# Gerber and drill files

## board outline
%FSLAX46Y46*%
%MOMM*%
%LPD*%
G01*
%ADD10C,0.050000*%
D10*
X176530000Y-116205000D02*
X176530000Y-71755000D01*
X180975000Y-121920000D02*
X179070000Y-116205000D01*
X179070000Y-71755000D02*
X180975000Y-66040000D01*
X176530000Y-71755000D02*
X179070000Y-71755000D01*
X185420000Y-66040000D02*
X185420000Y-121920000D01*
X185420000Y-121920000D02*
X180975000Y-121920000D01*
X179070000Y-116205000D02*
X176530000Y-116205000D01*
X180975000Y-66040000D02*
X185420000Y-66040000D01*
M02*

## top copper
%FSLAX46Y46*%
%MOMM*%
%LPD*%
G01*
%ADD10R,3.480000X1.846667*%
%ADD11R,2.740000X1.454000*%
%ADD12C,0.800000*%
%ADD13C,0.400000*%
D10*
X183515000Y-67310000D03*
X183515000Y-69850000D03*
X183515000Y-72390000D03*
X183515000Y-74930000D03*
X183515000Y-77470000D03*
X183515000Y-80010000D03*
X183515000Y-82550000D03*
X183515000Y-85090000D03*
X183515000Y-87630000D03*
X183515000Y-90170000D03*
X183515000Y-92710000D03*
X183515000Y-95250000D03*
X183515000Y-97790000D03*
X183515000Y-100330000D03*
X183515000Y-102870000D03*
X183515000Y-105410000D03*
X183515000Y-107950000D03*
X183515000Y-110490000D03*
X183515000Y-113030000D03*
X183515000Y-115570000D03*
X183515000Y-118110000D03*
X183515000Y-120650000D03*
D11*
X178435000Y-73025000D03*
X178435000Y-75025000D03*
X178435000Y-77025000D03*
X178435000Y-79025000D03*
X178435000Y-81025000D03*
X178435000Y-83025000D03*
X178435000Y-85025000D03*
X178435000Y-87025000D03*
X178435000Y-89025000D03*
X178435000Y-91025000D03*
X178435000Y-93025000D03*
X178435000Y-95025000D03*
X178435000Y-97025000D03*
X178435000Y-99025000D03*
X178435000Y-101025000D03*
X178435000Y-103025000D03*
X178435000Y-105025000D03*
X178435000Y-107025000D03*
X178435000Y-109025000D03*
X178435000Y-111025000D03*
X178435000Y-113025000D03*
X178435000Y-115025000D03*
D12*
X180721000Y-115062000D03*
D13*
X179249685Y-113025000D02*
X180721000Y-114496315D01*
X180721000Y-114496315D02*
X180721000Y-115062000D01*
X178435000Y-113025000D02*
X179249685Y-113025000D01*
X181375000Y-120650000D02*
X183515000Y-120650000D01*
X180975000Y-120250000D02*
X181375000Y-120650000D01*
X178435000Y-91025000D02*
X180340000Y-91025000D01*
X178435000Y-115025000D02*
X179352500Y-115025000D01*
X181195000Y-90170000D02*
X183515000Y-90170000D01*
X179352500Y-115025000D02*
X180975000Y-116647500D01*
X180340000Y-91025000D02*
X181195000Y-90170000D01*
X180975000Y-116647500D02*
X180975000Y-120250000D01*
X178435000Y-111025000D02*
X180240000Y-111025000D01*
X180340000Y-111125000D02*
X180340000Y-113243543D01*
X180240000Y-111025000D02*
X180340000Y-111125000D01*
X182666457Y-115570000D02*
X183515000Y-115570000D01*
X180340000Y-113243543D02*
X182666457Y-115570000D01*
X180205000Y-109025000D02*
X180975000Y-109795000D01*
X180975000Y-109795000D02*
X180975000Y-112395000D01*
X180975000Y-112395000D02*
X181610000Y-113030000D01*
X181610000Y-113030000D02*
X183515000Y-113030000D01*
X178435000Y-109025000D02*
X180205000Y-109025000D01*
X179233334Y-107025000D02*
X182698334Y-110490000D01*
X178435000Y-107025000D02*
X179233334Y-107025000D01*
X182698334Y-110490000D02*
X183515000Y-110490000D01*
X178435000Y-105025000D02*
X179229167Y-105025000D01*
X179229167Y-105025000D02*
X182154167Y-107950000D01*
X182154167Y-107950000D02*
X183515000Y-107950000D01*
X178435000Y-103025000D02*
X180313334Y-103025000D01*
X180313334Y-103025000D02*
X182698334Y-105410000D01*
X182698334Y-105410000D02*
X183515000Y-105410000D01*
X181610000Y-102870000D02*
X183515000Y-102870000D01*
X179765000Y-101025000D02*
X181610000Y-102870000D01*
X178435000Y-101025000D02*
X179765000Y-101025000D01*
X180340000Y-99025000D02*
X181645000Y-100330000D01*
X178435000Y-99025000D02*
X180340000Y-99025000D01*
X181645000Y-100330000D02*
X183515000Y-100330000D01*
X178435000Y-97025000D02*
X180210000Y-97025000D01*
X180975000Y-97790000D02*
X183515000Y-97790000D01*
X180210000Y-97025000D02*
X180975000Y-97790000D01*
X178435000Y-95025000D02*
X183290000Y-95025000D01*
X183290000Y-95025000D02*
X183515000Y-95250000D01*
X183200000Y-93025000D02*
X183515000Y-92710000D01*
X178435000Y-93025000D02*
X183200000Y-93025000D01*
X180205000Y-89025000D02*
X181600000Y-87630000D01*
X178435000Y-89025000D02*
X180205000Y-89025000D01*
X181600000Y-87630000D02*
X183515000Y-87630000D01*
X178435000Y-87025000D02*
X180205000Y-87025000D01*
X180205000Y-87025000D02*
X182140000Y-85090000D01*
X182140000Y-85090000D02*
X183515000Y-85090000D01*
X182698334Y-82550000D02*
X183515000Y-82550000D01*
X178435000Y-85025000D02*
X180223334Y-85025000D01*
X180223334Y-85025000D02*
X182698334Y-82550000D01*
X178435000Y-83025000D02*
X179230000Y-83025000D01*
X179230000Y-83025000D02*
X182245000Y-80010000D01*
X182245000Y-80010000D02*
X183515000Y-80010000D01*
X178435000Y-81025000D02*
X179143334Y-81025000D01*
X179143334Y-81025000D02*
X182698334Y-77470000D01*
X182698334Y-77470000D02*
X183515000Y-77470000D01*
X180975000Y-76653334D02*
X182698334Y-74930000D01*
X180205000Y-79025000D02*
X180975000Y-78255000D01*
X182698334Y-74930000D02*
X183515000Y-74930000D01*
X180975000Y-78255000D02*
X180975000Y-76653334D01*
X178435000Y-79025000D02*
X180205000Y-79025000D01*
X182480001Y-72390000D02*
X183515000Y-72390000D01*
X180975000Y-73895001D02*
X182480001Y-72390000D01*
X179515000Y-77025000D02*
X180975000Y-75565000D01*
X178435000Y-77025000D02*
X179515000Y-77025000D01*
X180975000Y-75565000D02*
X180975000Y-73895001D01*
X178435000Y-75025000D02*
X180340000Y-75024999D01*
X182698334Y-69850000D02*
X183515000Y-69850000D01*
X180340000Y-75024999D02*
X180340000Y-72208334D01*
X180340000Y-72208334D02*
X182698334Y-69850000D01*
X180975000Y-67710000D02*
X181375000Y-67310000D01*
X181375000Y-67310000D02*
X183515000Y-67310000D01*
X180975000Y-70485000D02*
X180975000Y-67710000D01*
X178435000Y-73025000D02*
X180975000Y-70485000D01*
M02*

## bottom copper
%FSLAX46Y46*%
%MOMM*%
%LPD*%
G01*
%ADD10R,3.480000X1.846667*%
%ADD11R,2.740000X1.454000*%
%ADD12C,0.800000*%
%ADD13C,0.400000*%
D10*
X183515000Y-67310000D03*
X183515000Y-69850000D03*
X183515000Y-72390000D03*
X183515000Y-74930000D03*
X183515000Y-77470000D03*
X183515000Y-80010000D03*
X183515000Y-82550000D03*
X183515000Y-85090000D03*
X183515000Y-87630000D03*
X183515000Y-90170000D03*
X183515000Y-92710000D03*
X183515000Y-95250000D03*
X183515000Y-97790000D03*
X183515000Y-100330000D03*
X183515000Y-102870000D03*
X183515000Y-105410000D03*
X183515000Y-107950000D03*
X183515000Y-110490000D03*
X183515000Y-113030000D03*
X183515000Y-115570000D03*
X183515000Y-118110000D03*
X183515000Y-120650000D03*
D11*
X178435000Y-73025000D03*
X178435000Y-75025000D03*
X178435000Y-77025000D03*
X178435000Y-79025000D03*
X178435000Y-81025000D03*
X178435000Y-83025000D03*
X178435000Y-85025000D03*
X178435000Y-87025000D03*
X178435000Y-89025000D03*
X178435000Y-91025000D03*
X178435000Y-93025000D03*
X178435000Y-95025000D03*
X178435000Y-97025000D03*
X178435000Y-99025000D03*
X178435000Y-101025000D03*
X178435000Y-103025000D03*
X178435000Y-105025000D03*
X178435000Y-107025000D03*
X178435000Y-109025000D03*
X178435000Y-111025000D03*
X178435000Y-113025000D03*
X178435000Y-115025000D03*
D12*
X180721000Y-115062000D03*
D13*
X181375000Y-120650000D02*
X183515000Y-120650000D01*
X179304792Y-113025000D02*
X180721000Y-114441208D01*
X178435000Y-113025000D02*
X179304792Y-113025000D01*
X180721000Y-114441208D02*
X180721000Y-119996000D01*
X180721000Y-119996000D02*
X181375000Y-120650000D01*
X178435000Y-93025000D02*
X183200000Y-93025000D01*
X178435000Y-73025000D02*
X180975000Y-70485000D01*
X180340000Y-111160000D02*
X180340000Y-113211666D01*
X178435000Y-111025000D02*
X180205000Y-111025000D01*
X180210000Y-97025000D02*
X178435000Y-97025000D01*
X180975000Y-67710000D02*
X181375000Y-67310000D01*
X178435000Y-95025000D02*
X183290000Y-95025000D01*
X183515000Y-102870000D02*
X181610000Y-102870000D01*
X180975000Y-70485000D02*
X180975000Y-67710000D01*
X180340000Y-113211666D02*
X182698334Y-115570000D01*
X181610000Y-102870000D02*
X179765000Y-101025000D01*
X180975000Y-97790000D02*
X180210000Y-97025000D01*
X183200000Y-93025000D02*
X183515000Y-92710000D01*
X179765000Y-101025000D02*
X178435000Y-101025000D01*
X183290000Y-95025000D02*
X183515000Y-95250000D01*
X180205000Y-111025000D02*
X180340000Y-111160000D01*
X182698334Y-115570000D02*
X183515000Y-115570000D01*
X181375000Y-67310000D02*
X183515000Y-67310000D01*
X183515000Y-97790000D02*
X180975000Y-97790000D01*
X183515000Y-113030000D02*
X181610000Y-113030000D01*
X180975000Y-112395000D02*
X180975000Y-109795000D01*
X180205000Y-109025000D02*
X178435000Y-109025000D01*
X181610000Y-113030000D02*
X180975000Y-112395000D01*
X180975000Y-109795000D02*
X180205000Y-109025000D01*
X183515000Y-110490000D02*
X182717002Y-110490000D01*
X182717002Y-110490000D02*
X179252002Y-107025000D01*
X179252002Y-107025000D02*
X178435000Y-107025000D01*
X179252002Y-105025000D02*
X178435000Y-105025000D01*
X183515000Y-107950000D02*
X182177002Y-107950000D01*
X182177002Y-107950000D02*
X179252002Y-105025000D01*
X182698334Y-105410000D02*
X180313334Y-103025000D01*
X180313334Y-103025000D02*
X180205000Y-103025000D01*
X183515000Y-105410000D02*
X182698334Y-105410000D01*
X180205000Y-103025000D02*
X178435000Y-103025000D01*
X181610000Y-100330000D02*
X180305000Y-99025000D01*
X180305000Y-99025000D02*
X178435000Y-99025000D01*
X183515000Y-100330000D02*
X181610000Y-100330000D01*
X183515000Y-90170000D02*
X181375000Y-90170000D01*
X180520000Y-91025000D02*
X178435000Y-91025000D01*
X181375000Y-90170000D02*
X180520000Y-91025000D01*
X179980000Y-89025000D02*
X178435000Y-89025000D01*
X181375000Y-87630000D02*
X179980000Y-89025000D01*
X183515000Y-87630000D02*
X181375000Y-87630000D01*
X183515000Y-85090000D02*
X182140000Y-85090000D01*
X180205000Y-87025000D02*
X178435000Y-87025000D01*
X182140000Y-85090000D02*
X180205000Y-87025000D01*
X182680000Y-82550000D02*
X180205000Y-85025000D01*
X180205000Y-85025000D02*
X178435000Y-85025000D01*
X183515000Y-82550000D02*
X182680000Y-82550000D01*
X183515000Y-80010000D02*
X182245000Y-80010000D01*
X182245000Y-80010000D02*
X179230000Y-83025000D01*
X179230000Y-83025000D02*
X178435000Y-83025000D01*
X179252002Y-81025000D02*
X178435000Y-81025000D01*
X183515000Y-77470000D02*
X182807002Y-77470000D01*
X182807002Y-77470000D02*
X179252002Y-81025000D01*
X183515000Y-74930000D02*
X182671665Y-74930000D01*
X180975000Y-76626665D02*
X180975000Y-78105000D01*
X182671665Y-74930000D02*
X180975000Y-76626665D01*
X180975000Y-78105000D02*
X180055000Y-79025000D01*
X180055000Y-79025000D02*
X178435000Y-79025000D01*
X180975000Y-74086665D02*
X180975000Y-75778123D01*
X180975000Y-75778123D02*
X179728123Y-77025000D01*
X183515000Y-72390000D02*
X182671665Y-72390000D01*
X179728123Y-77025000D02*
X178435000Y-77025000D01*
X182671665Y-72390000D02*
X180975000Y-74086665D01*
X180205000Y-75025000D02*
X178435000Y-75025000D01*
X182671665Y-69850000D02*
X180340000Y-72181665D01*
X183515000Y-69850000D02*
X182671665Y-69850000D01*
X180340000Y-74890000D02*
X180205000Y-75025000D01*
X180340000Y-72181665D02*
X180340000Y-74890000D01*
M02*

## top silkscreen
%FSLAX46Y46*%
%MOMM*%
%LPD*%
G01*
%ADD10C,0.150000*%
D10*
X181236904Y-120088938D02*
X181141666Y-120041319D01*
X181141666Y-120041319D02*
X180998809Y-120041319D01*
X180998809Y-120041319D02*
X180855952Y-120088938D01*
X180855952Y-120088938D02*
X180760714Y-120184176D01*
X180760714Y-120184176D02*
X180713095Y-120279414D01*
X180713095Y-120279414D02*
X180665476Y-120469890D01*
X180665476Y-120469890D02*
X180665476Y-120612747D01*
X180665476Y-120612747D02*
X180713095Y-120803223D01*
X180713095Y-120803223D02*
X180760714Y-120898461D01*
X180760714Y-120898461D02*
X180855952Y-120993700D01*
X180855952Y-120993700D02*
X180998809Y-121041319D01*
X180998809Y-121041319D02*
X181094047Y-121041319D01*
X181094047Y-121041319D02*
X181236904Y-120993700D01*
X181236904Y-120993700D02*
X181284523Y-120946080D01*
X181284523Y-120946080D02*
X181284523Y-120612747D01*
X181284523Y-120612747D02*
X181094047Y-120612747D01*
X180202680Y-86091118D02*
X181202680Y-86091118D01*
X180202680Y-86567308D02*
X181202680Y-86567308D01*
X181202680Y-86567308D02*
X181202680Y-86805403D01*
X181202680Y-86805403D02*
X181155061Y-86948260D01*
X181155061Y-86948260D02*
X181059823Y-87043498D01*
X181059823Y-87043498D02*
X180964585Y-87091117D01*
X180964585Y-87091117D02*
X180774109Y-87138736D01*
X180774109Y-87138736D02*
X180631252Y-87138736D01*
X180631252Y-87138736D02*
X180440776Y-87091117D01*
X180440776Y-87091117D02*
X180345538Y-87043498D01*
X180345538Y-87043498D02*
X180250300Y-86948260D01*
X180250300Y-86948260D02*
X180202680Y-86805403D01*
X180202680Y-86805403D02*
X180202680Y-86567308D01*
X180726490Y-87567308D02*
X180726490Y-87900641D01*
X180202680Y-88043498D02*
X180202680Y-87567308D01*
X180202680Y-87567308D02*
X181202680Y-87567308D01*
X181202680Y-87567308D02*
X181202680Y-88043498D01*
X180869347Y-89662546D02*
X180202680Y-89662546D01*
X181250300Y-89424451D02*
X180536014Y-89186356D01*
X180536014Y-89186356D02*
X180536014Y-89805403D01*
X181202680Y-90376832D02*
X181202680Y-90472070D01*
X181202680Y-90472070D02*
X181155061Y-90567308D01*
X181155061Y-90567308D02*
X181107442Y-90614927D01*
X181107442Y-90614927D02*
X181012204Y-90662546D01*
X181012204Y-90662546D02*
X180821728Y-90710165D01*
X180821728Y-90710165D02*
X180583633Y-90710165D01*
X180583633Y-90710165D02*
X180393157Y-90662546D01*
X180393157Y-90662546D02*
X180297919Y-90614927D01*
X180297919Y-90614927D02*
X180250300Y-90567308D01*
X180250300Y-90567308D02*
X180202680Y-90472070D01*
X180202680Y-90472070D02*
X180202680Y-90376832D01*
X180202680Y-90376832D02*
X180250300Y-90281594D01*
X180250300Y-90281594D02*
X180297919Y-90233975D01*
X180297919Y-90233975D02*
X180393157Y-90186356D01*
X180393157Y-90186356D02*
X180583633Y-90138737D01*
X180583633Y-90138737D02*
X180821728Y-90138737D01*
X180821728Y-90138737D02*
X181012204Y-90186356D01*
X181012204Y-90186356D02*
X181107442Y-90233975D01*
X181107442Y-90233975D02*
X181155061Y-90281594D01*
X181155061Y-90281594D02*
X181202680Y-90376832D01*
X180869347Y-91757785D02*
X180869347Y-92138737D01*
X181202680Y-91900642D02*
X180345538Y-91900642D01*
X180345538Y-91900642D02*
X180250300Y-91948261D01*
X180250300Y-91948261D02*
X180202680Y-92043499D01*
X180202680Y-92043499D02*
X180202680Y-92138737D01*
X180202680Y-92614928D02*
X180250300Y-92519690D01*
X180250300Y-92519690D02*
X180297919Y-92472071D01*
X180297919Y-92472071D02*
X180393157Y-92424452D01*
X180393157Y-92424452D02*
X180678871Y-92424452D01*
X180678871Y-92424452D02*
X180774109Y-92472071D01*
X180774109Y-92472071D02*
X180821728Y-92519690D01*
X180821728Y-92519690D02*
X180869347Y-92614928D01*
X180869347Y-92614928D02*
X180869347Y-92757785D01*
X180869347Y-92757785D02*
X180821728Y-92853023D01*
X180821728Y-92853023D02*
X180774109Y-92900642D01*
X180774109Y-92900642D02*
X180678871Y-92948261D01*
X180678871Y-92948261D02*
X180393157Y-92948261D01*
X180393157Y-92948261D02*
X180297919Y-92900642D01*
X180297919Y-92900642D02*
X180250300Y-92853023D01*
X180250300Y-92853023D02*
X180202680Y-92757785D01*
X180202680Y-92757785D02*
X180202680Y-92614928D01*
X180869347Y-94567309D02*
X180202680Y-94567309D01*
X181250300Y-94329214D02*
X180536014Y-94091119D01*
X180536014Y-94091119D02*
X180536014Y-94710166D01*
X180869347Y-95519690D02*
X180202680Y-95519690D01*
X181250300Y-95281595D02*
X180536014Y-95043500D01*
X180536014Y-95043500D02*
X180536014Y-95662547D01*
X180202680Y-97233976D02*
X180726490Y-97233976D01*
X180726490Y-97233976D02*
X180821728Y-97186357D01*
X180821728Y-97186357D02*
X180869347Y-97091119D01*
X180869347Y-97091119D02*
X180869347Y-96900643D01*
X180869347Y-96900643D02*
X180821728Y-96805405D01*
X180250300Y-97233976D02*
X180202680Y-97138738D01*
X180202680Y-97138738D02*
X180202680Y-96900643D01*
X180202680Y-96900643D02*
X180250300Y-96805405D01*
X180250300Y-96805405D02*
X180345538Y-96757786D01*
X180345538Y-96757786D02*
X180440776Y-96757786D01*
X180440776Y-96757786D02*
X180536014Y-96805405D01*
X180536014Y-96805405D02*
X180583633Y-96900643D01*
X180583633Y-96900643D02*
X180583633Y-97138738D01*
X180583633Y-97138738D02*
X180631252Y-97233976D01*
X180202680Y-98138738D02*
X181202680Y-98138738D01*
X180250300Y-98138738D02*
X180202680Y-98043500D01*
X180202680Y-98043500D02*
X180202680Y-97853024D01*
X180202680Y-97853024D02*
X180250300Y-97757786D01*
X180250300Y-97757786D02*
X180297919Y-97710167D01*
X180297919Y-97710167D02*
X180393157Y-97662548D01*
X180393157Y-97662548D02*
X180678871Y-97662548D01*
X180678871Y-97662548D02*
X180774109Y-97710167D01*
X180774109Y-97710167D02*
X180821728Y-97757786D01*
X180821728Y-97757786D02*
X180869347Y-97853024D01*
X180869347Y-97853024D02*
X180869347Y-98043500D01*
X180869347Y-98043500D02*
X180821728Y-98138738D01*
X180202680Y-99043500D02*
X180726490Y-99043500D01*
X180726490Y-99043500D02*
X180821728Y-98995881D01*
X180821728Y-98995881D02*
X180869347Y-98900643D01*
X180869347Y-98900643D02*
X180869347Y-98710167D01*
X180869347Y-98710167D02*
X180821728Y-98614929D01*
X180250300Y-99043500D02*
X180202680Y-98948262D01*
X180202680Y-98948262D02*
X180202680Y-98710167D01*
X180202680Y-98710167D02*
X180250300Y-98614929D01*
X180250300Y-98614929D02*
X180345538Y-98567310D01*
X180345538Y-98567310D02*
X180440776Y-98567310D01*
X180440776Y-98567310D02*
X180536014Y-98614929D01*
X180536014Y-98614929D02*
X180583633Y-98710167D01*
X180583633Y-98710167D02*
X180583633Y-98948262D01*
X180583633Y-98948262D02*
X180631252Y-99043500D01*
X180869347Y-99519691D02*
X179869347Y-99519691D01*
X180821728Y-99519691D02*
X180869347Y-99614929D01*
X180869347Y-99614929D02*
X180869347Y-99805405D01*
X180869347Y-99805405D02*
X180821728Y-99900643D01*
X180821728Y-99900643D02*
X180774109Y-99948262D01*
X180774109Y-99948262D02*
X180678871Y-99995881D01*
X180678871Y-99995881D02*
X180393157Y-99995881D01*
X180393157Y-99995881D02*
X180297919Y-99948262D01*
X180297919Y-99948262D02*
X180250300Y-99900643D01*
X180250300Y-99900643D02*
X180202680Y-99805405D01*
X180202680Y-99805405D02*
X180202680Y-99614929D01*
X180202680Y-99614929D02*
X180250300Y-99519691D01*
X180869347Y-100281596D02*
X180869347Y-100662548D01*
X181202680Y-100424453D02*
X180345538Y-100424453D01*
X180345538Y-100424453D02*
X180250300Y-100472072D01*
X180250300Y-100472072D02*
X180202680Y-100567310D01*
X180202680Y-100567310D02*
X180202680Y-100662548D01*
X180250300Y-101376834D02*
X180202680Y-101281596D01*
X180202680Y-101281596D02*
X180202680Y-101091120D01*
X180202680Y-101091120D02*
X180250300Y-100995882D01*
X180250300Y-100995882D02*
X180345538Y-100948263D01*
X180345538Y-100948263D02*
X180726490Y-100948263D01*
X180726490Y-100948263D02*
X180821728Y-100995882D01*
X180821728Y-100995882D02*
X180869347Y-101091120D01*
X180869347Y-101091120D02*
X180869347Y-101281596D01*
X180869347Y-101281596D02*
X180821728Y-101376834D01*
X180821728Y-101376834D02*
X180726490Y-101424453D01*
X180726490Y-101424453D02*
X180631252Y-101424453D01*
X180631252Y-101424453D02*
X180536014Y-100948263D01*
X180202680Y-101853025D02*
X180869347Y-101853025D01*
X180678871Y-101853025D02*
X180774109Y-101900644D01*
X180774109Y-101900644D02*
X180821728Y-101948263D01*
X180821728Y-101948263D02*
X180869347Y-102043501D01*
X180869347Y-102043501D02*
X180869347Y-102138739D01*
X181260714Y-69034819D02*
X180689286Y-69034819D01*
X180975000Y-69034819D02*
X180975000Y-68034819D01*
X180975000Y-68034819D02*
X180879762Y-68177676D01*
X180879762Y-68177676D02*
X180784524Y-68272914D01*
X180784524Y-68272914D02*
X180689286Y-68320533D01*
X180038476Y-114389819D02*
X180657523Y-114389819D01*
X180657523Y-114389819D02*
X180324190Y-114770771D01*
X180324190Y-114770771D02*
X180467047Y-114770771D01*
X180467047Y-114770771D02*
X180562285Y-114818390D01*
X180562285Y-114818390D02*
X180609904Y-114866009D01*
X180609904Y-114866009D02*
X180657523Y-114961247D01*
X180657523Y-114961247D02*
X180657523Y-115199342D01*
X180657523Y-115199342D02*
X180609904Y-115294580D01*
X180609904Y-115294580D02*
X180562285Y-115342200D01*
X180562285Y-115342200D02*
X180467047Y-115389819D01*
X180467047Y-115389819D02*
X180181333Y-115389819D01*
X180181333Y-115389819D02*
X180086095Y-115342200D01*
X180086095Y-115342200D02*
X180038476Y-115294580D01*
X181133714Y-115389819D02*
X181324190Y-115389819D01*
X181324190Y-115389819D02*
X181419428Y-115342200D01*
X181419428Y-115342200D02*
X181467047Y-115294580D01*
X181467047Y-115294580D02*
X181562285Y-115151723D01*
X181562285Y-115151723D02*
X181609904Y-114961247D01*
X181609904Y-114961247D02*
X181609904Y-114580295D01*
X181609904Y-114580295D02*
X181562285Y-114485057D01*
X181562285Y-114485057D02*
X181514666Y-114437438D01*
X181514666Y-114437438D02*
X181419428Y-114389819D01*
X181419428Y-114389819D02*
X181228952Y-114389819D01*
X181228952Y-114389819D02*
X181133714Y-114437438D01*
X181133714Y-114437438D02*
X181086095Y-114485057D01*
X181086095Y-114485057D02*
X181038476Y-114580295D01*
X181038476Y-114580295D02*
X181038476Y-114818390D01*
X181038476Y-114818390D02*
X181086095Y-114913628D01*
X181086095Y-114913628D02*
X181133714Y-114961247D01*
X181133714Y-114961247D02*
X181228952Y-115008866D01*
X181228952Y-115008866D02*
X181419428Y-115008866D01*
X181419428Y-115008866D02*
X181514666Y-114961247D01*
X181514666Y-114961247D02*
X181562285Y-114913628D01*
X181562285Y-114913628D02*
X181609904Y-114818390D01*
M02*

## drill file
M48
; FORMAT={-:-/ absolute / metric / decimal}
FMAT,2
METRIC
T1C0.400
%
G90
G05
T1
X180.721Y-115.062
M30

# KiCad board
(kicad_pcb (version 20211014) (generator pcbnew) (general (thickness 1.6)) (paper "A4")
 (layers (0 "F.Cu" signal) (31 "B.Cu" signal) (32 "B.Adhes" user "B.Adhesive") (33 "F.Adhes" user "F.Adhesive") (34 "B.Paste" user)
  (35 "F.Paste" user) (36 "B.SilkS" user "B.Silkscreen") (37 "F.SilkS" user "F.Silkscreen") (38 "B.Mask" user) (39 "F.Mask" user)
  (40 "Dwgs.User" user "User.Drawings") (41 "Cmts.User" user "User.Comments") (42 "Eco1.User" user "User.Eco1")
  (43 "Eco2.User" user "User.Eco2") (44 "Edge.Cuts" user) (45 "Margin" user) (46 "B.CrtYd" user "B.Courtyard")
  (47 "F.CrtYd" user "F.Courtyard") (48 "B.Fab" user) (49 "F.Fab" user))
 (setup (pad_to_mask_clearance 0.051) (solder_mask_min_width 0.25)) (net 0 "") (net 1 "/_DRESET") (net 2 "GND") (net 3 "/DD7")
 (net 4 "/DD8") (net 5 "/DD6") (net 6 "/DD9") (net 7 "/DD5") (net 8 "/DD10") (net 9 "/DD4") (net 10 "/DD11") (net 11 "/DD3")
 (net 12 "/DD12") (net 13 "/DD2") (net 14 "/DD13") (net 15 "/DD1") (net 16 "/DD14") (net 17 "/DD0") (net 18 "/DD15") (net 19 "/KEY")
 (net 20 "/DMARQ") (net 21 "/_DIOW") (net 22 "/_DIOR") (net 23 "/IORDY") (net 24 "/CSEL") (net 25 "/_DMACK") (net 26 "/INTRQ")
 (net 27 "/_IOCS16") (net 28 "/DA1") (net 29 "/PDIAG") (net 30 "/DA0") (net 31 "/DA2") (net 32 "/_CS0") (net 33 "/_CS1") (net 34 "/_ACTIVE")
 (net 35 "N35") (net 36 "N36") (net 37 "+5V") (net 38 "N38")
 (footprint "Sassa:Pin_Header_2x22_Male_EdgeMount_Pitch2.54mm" (layer "B.Cu") (at 183.515 67.31 -90)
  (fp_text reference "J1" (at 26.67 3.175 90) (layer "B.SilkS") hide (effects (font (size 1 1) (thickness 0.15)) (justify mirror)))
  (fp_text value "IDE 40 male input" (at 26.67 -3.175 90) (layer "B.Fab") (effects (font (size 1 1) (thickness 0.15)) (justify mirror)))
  (pad "1" smd rect locked (at 0 0 270) (size 1.846667 3.48) (layers "F.Cu" "F.Paste" "F.Mask") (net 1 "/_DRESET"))
  (pad "2" smd rect locked (at 0 0 270) (size 1.846667 3.48) (layers "B.Cu" "B.Paste" "B.Mask") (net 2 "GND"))
  (pad "3" smd rect locked (at 2.54 0 270) (size 1.846667 3.48) (layers "F.Cu" "F.Paste" "F.Mask") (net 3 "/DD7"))
  (pad "4" smd rect locked (at 2.54 0 270) (size 1.846667 3.48) (layers "B.Cu" "B.Paste" "B.Mask") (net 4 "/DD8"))
  (pad "5" smd rect locked (at 5.08 0 270) (size 1.846667 3.48) (layers "F.Cu" "F.Paste" "F.Mask") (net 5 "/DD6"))
  (pad "6" smd rect locked (at 5.08 0 270) (size 1.846667 3.48) (layers "B.Cu" "B.Paste" "B.Mask") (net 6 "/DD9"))
  (pad "7" smd rect locked (at 7.62 0 270) (size 1.846667 3.48) (layers "F.Cu" "F.Paste" "F.Mask") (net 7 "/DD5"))
  (pad "8" smd rect locked (at 7.62 0 270) (size 1.846667 3.48) (layers "B.Cu" "B.Paste" "B.Mask") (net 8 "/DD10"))
  (pad "9" smd rect locked (at 10.16 0 270) (size 1.846667 3.48) (layers "F.Cu" "F.Paste" "F.Mask") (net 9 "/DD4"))
  (pad "10" smd rect locked (at 10.16 0 270) (size 1.846667 3.48) (layers "B.Cu" "B.Paste" "B.Mask") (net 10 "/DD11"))
  (pad "11" smd rect locked (at 12.7 0 270) (size 1.846667 3.48) (layers "F.Cu" "F.Paste" "F.Mask") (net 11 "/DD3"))
  (pad "12" smd rect locked (at 12.7 0 270) (size 1.846667 3.48) (layers "B.Cu" "B.Paste" "B.Mask") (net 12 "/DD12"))
  (pad "13" smd rect locked (at 15.24 0 270) (size 1.846667 3.48) (layers "F.Cu" "F.Paste" "F.Mask") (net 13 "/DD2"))
  (pad "14" smd rect locked (at 15.24 0 270) (size 1.846667 3.48) (layers "B.Cu" "B.Paste" "B.Mask") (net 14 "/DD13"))
  (pad "15" smd rect locked (at 17.78 0 270) (size 1.846667 3.48) (layers "F.Cu" "F.Paste" "F.Mask") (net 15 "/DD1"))
  (pad "16" smd rect locked (at 17.78 0 270) (size 1.846667 3.48) (layers "B.Cu" "B.Paste" "B.Mask") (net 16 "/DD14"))
  (pad "17" smd rect locked (at 20.32 0 270) (size 1.846667 3.48) (layers "F.Cu" "F.Paste" "F.Mask") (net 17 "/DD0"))
  (pad "18" smd rect locked (at 20.32 0 270) (size 1.846667 3.48) (layers "B.Cu" "B.Paste" "B.Mask") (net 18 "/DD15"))
  (pad "19" smd rect locked (at 22.86 0 270) (size 1.846667 3.48) (layers "F.Cu" "F.Paste" "F.Mask") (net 2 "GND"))
  (pad "20" smd rect locked (at 22.86 0 270) (size 1.846667 3.48) (layers "B.Cu" "B.Paste" "B.Mask") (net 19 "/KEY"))
  (pad "21" smd rect locked (at 25.4 0 270) (size 1.846667 3.48) (layers "F.Cu" "F.Paste" "F.Mask") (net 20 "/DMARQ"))
  (pad "22" smd rect locked (at 25.4 0 270) (size 1.846667 3.48) (layers "B.Cu" "B.Paste" "B.Mask") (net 2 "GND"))
  (pad "23" smd rect locked (at 27.94 0 270) (size 1.846667 3.48) (layers "F.Cu" "F.Paste" "F.Mask") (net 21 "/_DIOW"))
  (pad "24" smd rect locked (at 27.94 0 270) (size 1.846667 3.48) (layers "B.Cu" "B.Paste" "B.Mask") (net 2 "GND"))
  (pad "25" smd rect locked (at 30.48 0 270) (size 1.846667 3.48) (layers "F.Cu" "F.Paste" "F.Mask") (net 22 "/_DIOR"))
  (pad "26" smd rect locked (at 30.48 0 270) (size 1.846667 3.48) (layers "B.Cu" "B.Paste" "B.Mask") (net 2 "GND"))
  (pad "27" smd rect locked (at 33.02 0 270) (size 1.846667 3.48) (layers "F.Cu" "F.Paste" "F.Mask") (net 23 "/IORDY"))
  (pad "28" smd rect locked (at 33.02 0 270) (size 1.846667 3.48) (layers "B.Cu" "B.Paste" "B.Mask") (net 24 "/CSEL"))
  (pad "29" smd rect locked (at 35.56 0 270) (size 1.846667 3.48) (layers "F.Cu" "F.Paste" "F.Mask") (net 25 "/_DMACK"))
  (pad "30" smd rect locked (at 35.56 0 270) (size 1.846667 3.48) (layers "B.Cu" "B.Paste" "B.Mask") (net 2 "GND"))
  (pad "31" smd rect locked (at 38.1 0 270) (size 1.846667 3.48) (layers "F.Cu" "F.Paste" "F.Mask") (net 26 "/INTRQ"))
  (pad "32" smd rect locked (at 38.1 0 270) (size 1.846667 3.48) (layers "B.Cu" "B.Paste" "B.Mask") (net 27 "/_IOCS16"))
  (pad "33" smd rect locked (at 40.64 0 270) (size 1.846667 3.48) (layers "F.Cu" "F.Paste" "F.Mask") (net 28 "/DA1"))
  (pad "34" smd rect locked (at 40.64 0 270) (size 1.846667 3.48) (layers "B.Cu" "B.Paste" "B.Mask") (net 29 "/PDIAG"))
  (pad "35" smd rect locked (at 43.18 0 270) (size 1.846667 3.48) (layers "F.Cu" "F.Paste" "F.Mask") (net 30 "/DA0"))
  (pad "36" smd rect locked (at 43.18 0 270) (size 1.846667 3.48) (layers "B.Cu" "B.Paste" "B.Mask") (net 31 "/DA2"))
  (pad "37" smd rect locked (at 45.72 0 270) (size 1.846667 3.48) (layers "F.Cu" "F.Paste" "F.Mask") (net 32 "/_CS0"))
  (pad "38" smd rect locked (at 45.72 0 270) (size 1.846667 3.48) (layers "B.Cu" "B.Paste" "B.Mask") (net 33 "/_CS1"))
  (pad "39" smd rect locked (at 48.26 0 270) (size 1.846667 3.48) (layers "F.Cu" "F.Paste" "F.Mask") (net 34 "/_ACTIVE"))
  (pad "40" smd rect locked (at 48.26 0 270) (size 1.846667 3.48) (layers "B.Cu" "B.Paste" "B.Mask") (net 2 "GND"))
  (pad "41" smd rect locked (at 50.8 0 270) (size 1.846667 3.48) (layers "F.Cu" "F.Paste" "F.Mask") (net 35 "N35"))
  (pad "42" smd rect locked (at 50.8 0 270) (size 1.846667 3.48) (layers "B.Cu" "B.Paste" "B.Mask") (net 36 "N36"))
  (pad "43" smd rect locked (at 53.34 0 270) (size 1.846667 3.48) (layers "F.Cu" "F.Paste" "F.Mask") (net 2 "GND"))
  (pad "44" smd rect locked (at 53.34 0 270) (size 1.846667 3.48) (layers "B.Cu" "B.Paste" "B.Mask") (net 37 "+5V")))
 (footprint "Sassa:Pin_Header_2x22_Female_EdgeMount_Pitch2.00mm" (layer "B.Cu") (at 178.435 73.025 90)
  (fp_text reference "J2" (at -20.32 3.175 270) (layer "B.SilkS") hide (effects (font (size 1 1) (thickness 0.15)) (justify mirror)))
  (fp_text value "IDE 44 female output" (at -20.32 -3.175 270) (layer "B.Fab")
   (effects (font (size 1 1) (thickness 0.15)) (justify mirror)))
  (pad "1" smd rect locked (at 0 0 90) (size 1.454 2.74) (layers "F.Cu" "F.Paste" "F.Mask") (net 1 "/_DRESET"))
  (pad "2" smd rect locked (at 0 0 90) (size 1.454 2.74) (layers "B.Cu" "B.Paste" "B.Mask") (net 2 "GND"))
  (pad "3" smd rect locked (at -2 0 90) (size 1.454 2.74) (layers "F.Cu" "F.Paste" "F.Mask") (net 3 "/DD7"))
  (pad "4" smd rect locked (at -2 0 90) (size 1.454 2.74) (layers "B.Cu" "B.Paste" "B.Mask") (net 4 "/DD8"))
  (pad "5" smd rect locked (at -4 0 90) (size 1.454 2.74) (layers "F.Cu" "F.Paste" "F.Mask") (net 5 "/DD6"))
  (pad "6" smd rect locked (at -4 0 90) (size 1.454 2.74) (layers "B.Cu" "B.Paste" "B.Mask") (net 6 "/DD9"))
  (pad "7" smd rect locked (at -6 0 90) (size 1.454 2.74) (layers "F.Cu" "F.Paste" "F.Mask") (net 7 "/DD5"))
  (pad "8" smd rect locked (at -6 0 90) (size 1.454 2.74) (layers "B.Cu" "B.Paste" "B.Mask") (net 8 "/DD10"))
  (pad "9" smd rect locked (at -8 0 90) (size 1.454 2.74) (layers "F.Cu" "F.Paste" "F.Mask") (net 9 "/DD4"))
  (pad "10" smd rect locked (at -8 0 90) (size 1.454 2.74) (layers "B.Cu" "B.Paste" "B.Mask") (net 10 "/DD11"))
  (pad "11" smd rect locked (at -10 0 90) (size 1.454 2.74) (layers "F.Cu" "F.Paste" "F.Mask") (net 11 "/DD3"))
  (pad "12" smd rect locked (at -10 0 90) (size 1.454 2.74) (layers "B.Cu" "B.Paste" "B.Mask") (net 12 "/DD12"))
  (pad "13" smd rect locked (at -12 0 90) (size 1.454 2.74) (layers "F.Cu" "F.Paste" "F.Mask") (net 13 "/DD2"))
  (pad "14" smd rect locked (at -12 0 90) (size 1.454 2.74) (layers "B.Cu" "B.Paste" "B.Mask") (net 14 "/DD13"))
  (pad "15" smd rect locked (at -14 0 90) (size 1.454 2.74) (layers "F.Cu" "F.Paste" "F.Mask") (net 15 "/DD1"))
  (pad "16" smd rect locked (at -14 0 90) (size 1.454 2.74) (layers "B.Cu" "B.Paste" "B.Mask") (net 16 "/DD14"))
  (pad "17" smd rect locked (at -16 0 90) (size 1.454 2.74) (layers "F.Cu" "F.Paste" "F.Mask") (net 17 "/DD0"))
  (pad "18" smd rect locked (at -16 0 90) (size 1.454 2.74) (layers "B.Cu" "B.Paste" "B.Mask") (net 18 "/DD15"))
  (pad "19" smd rect locked (at -18 0 90) (size 1.454 2.74) (layers "F.Cu" "F.Paste" "F.Mask") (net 2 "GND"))
  (pad "20" smd rect locked (at -18 0 90) (size 1.454 2.74) (layers "B.Cu" "B.Paste" "B.Mask") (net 19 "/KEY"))
  (pad "21" smd rect locked (at -20 0 90) (size 1.454 2.74) (layers "F.Cu" "F.Paste" "F.Mask") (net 20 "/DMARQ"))
  (pad "22" smd rect locked (at -20 0 90) (size 1.454 2.74) (layers "B.Cu" "B.Paste" "B.Mask") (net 2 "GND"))
  (pad "23" smd rect locked (at -22 0 90) (size 1.454 2.74) (layers "F.Cu" "F.Paste" "F.Mask") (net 21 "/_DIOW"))
  (pad "24" smd rect locked (at -22 0 90) (size 1.454 2.74) (layers "B.Cu" "B.Paste" "B.Mask") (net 2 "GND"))
  (pad "25" smd rect locked (at -24 0 90) (size 1.454 2.74) (layers "F.Cu" "F.Paste" "F.Mask") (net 22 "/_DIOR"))
  (pad "26" smd rect locked (at -24 0 90) (size 1.454 2.74) (layers "B.Cu" "B.Paste" "B.Mask") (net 2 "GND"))
  (pad "27" smd rect locked (at -26 0 90) (size 1.454 2.74) (layers "F.Cu" "F.Paste" "F.Mask") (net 23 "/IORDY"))
  (pad "28" smd rect locked (at -26 0 90) (size 1.454 2.74) (layers "B.Cu" "B.Paste" "B.Mask") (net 24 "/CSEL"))
  (pad "29" smd rect locked (at -28 0 90) (size 1.454 2.74) (layers "F.Cu" "F.Paste" "F.Mask") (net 25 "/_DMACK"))
  (pad "30" smd rect locked (at -28 0 90) (size 1.454 2.74) (layers "B.Cu" "B.Paste" "B.Mask") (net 2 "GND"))
  (pad "31" smd rect locked (at -30 0 90) (size 1.454 2.74) (layers "F.Cu" "F.Paste" "F.Mask") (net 26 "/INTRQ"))
  (pad "32" smd rect locked (at -30 0 90) (size 1.454 2.74) (layers "B.Cu" "B.Paste" "B.Mask") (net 27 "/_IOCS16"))
  (pad "33" smd rect locked (at -32 0 90) (size 1.454 2.74) (layers "F.Cu" "F.Paste" "F.Mask") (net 28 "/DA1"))
  (pad "34" smd rect locked (at -32 0 90) (size 1.454 2.74) (layers "B.Cu" "B.Paste" "B.Mask") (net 29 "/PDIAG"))
  (pad "35" smd rect locked (at -34 0 90) (size 1.454 2.74) (layers "F.Cu" "F.Paste" "F.Mask") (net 30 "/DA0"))
  (pad "36" smd rect locked (at -34 0 90) (size 1.454 2.74) (layers "B.Cu" "B.Paste" "B.Mask") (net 31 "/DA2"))
  (pad "37" smd rect locked (at -36 0 90) (size 1.454 2.74) (layers "F.Cu" "F.Paste" "F.Mask") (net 32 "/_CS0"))
  (pad "38" smd rect locked (at -36 0 90) (size 1.454 2.74) (layers "B.Cu" "B.Paste" "B.Mask") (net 33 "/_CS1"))
  (pad "39" smd rect locked (at -38 0 90) (size 1.454 2.74) (layers "F.Cu" "F.Paste" "F.Mask") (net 34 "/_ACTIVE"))
  (pad "40" smd rect locked (at -38 0 90) (size 1.454 2.74) (layers "B.Cu" "B.Paste" "B.Mask") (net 2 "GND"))
  (pad "41" smd rect locked (at -40 0 90) (size 1.454 2.74) (layers "F.Cu" "F.Paste" "F.Mask") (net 37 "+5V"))
  (pad "42" smd rect locked (at -40 0 90) (size 1.454 2.74) (layers "B.Cu" "B.Paste" "B.Mask") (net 37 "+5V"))
  (pad "43" smd rect locked (at -42 0 90) (size 1.454 2.74) (layers "F.Cu" "F.Paste" "F.Mask") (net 2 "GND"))
  (pad "44" smd rect locked (at -42 0 90) (size 1.454 2.74) (layers "B.Cu" "B.Paste" "B.Mask") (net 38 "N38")))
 (gr_line (start 176.53 116.205) (end 176.53 71.755) (layer "Edge.Cuts") (width 0.05))
 (gr_line (start 180.975 121.92) (end 179.07 116.205) (layer "Edge.Cuts") (width 0.05))
 (gr_line (start 179.07 71.755) (end 180.975 66.04) (layer "Edge.Cuts") (width 0.05))
 (gr_line (start 176.53 71.755) (end 179.07 71.755) (layer "Edge.Cuts") (width 0.05))
 (gr_line (start 185.42 66.04) (end 185.42 121.92) (layer "Edge.Cuts") (width 0.05))
 (gr_line (start 185.42 121.92) (end 180.975 121.92) (layer "Edge.Cuts") (width 0.05))
 (gr_line (start 179.07 116.205) (end 176.53 116.205) (layer "Edge.Cuts") (width 0.05))
 (gr_line (start 180.975 66.04) (end 185.42 66.04) (layer "Edge.Cuts") (width 0.05))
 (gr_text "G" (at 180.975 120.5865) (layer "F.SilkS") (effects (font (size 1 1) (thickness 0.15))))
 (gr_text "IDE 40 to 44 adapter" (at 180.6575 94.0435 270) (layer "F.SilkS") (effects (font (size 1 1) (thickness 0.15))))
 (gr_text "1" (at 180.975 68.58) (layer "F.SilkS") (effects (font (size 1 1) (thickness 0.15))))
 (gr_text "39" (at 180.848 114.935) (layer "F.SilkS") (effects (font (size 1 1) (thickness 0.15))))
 (segment (start 179.249685 113.025) (end 180.721 114.496315) (width 0.4) (layer "F.Cu") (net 37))
 (segment (start 180.721 114.496315) (end 180.721 115.062) (width 0.4) (layer "F.Cu") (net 37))
 (segment (start 178.435 113.025) (end 179.249685 113.025) (width 0.4) (layer "F.Cu") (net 37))
 (via (at 180.721 115.062) (size 0.8) (drill 0.4) (layers "F.Cu" "B.Cu") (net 37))
 (segment (start 181.375 120.65) (end 183.515 120.65) (width 0.4) (layer "B.Cu") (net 37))
 (segment (start 179.304792 113.025) (end 180.721 114.441208) (width 0.4) (layer "B.Cu") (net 37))
 (segment (start 178.435 113.025) (end 179.304792 113.025) (width 0.4) (layer "B.Cu") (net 37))
 (segment (start 180.721 114.441208) (end 180.721 119.996) (width 0.4) (layer "B.Cu") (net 37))
 (segment (start 180.721 119.996) (end 181.375 120.65) (width 0.4) (layer "B.Cu") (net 37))
 (segment (start 181.375 120.65) (end 183.515 120.65) (width 0.4) (layer "F.Cu") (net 2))
 (segment (start 180.975 120.25) (end 181.375 120.65) (width 0.4) (layer "F.Cu") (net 2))
 (segment (start 178.435 91.025) (end 180.34 91.025) (width 0.4) (layer "F.Cu") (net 2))
 (segment (start 178.435 115.025) (end 179.3525 115.025) (width 0.4) (layer "F.Cu") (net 2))
 (segment (start 181.195 90.17) (end 183.515 90.17) (width 0.4) (layer "F.Cu") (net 2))
 (segment (start 179.3525 115.025) (end 180.975 116.6475) (width 0.4) (layer "F.Cu") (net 2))
 (segment (start 180.34 91.025) (end 181.195 90.17) (width 0.4) (layer "F.Cu") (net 2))
 (segment (start 180.975 116.6475) (end 180.975 120.25) (width 0.4) (layer "F.Cu") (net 2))
 (segment (start 178.435 93.025) (end 183.2 93.025) (width 0.4) (layer "B.Cu") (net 2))
 (segment (start 178.435 73.025) (end 180.975 70.485) (width 0.4) (layer "B.Cu") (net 2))
 (segment (start 180.34 111.16) (end 180.34 113.211666) (width 0.4) (layer "B.Cu") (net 2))
 (segment (start 178.435 111.025) (end 180.205 111.025) (width 0.4) (layer "B.Cu") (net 2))
 (segment (start 180.21 97.025) (end 178.435 97.025) (width 0.4) (layer "B.Cu") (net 2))
 (segment (start 180.975 67.71) (end 181.375 67.31) (width 0.4) (layer "B.Cu") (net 2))
 (segment (start 178.435 95.025) (end 183.29 95.025) (width 0.4) (layer "B.Cu") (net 2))
 (segment (start 183.515 102.87) (end 181.61 102.87) (width 0.4) (layer "B.Cu") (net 2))
 (segment (start 180.975 70.485) (end 180.975 67.71) (width 0.4) (layer "B.Cu") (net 2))
 (segment (start 180.34 113.211666) (end 182.698334 115.57) (width 0.4) (layer "B.Cu") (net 2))
 (segment (start 181.61 102.87) (end 179.765 101.025) (width 0.4) (layer "B.Cu") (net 2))
 (segment (start 180.975 97.79) (end 180.21 97.025) (width 0.4) (layer "B.Cu") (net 2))
 (segment (start 183.2 93.025) (end 183.515 92.71) (width 0.4) (layer "B.Cu") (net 2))
 (segment (start 179.765 101.025) (end 178.435 101.025) (width 0.4) (layer "B.Cu") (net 2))
 (segment (start 183.29 95.025) (end 183.515 95.25) (width 0.4) (layer "B.Cu") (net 2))
 (segment (start 180.205 111.025) (end 180.34 111.16) (width 0.4) (layer "B.Cu") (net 2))
 (segment (start 182.698334 115.57) (end 183.515 115.57) (width 0.4) (layer "B.Cu") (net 2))
 (segment (start 181.375 67.31) (end 183.515 67.31) (width 0.4) (layer "B.Cu") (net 2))
 (segment (start 183.515 97.79) (end 180.975 97.79) (width 0.4) (layer "B.Cu") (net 2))
 (segment (start 183.515 113.03) (end 181.61 113.03) (width 0.4) (layer "B.Cu") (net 33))
 (segment (start 180.975 112.395) (end 180.975 109.795) (width 0.4) (layer "B.Cu") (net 33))
 (segment (start 180.205 109.025) (end 178.435 109.025) (width 0.4) (layer "B.Cu") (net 33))
 (segment (start 181.61 113.03) (end 180.975 112.395) (width 0.4) (layer "B.Cu") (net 33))
 (segment (start 180.975 109.795) (end 180.205 109.025) (width 0.4) (layer "B.Cu") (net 33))
 (segment (start 183.515 110.49) (end 182.717002 110.49) (width 0.4) (layer "B.Cu") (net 31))
 (segment (start 182.717002 110.49) (end 179.252002 107.025) (width 0.4) (layer "B.Cu") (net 31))
 (segment (start 179.252002 107.025) (end 178.435 107.025) (width 0.4) (layer "B.Cu") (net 31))
 (segment (start 179.252002 105.025) (end 178.435 105.025) (width 0.4) (layer "B.Cu") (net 29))
 (segment (start 183.515 107.95) (end 182.177002 107.95) (width 0.4) (layer "B.Cu") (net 29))
 (segment (start 182.177002 107.95) (end 179.252002 105.025) (width 0.4) (layer "B.Cu") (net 29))
 (segment (start 182.698334 105.41) (end 180.313334 103.025) (width 0.4) (layer "B.Cu") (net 27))
 (segment (start 180.313334 103.025) (end 180.205 103.025) (width 0.4) (layer "B.Cu") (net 27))
 (segment (start 183.515 105.41) (end 182.698334 105.41) (width 0.4) (layer "B.Cu") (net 27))
 (segment (start 180.205 103.025) (end 178.435 103.025) (width 0.4) (layer "B.Cu") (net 27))
 (segment (start 181.61 100.33) (end 180.305 99.025) (width 0.4) (layer "B.Cu") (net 24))
 (segment (start 180.305 99.025) (end 178.435 99.025) (width 0.4) (layer "B.Cu") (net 24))
 (segment (start 183.515 100.33) (end 181.61 100.33) (width 0.4) (layer "B.Cu") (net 24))
 (segment (start 183.515 90.17) (end 181.375 90.17) (width 0.4) (layer "B.Cu") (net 19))
 (segment (start 180.52 91.025) (end 178.435 91.025) (width 0.4) (layer "B.Cu") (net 19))
 (segment (start 181.375 90.17) (end 180.52 91.025) (width 0.4) (layer "B.Cu") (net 19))
 (segment (start 179.98 89.025) (end 178.435 89.025) (width 0.4) (layer "B.Cu") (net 18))
 (segment (start 181.375 87.63) (end 179.98 89.025) (width 0.4) (layer "B.Cu") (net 18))
 (segment (start 183.515 87.63) (end 181.375 87.63) (width 0.4) (layer "B.Cu") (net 18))
 (segment (start 183.515 85.09) (end 182.14 85.09) (width 0.4) (layer "B.Cu") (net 16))
 (segment (start 180.205 87.025) (end 178.435 87.025) (width 0.4) (layer "B.Cu") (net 16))
 (segment (start 182.14 85.09) (end 180.205 87.025) (width 0.4) (layer "B.Cu") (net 16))
 (segment (start 182.68 82.55) (end 180.205 85.025) (width 0.4) (layer "B.Cu") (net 14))
 (segment (start 180.205 85.025) (end 178.435 85.025) (width 0.4) (layer "B.Cu") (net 14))
 (segment (start 183.515 82.55) (end 182.68 82.55) (width 0.4) (layer "B.Cu") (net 14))
 (segment (start 183.515 80.01) (end 182.245 80.01) (width 0.4) (layer "B.Cu") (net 12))
 (segment (start 182.245 80.01) (end 179.23 83.025) (width 0.4) (layer "B.Cu") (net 12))
 (segment (start 179.23 83.025) (end 178.435 83.025) (width 0.4) (layer "B.Cu") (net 12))
 (segment (start 179.252002 81.025) (end 178.435 81.025) (width 0.4) (layer "B.Cu") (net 10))
 (segment (start 183.515 77.47) (end 182.807002 77.47) (width 0.4) (layer "B.Cu") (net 10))
 (segment (start 182.807002 77.47) (end 179.252002 81.025) (width 0.4) (layer "B.Cu") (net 10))
 (segment (start 183.515 74.93) (end 182.671665 74.93) (width 0.4) (layer "B.Cu") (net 8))
 (segment (start 180.975 76.626665) (end 180.975 78.105) (width 0.4) (layer "B.Cu") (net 8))
 (segment (start 182.671665 74.93) (end 180.975 76.626665) (width 0.4) (layer "B.Cu") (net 8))
 (segment (start 180.975 78.105) (end 180.055 79.025) (width 0.4) (layer "B.Cu") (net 8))
 (segment (start 180.055 79.025) (end 178.435 79.025) (width 0.4) (layer "B.Cu") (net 8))
 (segment (start 180.975 74.086665) (end 180.975 75.778123) (width 0.4) (layer "B.Cu") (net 6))
 (segment (start 180.975 75.778123) (end 179.728123 77.025) (width 0.4) (layer "B.Cu") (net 6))
 (segment (start 183.515 72.39) (end 182.671665 72.39) (width 0.4) (layer "B.Cu") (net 6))
 (segment (start 179.728123 77.025) (end 178.435 77.025) (width 0.4) (layer "B.Cu") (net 6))
 (segment (start 182.671665 72.39) (end 180.975 74.086665) (width 0.4) (layer "B.Cu") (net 6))
 (segment (start 180.205 75.025) (end 178.435 75.025) (width 0.4) (layer "B.Cu") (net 4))
 (segment (start 182.671665 69.85) (end 180.34 72.181665) (width 0.4) (layer "B.Cu") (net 4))
 (segment (start 183.515 69.85) (end 182.671665 69.85) (width 0.4) (layer "B.Cu") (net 4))
 (segment (start 180.34 74.89) (end 180.205 75.025) (width 0.4) (layer "B.Cu") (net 4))
 (segment (start 180.34 72.181665) (end 180.34 74.89) (width 0.4) (layer "B.Cu") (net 4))
 (segment (start 178.435 111.025) (end 180.24 111.025) (width 0.4) (layer "F.Cu") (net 34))
 (segment (start 180.34 111.125) (end 180.34 113.243543) (width 0.4) (layer "F.Cu") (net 34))
 (segment (start 180.24 111.025) (end 180.34 111.125) (width 0.4) (layer "F.Cu") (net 34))
 (segment (start 182.666457 115.57) (end 183.515 115.57) (width 0.4) (layer "F.Cu") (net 34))
 (segment (start 180.34 113.243543) (end 182.666457 115.57) (width 0.4) (layer "F.Cu") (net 34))
 (segment (start 180.205 109.025) (end 180.975 109.795) (width 0.4) (layer "F.Cu") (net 32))
 (segment (start 180.975 109.795) (end 180.975 112.395) (width 0.4) (layer "F.Cu") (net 32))
 (segment (start 180.975 112.395) (end 181.61 113.03) (width 0.4) (layer "F.Cu") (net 32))
 (segment (start 181.61 113.03) (end 183.515 113.03) (width 0.4) (layer "F.Cu") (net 32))
 (segment (start 178.435 109.025) (end 180.205 109.025) (width 0.4) (layer "F.Cu") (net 32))
 (segment (start 179.233334 107.025) (end 182.698334 110.49) (width 0.4) (layer "F.Cu") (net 30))
 (segment (start 178.435 107.025) (end 179.233334 107.025) (width 0.4) (layer "F.Cu") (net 30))
 (segment (start 182.698334 110.49) (end 183.515 110.49) (width 0.4) (layer "F.Cu") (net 30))
 (segment (start 178.435 105.025) (end 179.229167 105.025) (width 0.4) (layer "F.Cu") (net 28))
 (segment (start 179.229167 105.025) (end 182.154167 107.95) (width 0.4) (layer "F.Cu") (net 28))
 (segment (start 182.154167 107.95) (end 183.515 107.95) (width 0.4) (layer "F.Cu") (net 28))
 (segment (start 178.435 103.025) (end 180.313334 103.025) (width 0.4) (layer "F.Cu") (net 26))
 (segment (start 180.313334 103.025) (end 182.698334 105.41) (width 0.4) (layer "F.Cu") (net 26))
 (segment (start 182.698334 105.41) (end 183.515 105.41) (width 0.4) (layer "F.Cu") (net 26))
 (segment (start 181.61 102.87) (end 183.515 102.87) (width 0.4) (layer "F.Cu") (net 25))
 (segment (start 179.765 101.025) (end 181.61 102.87) (width 0.4) (layer "F.Cu") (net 25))
 (segment (start 178.435 101.025) (end 179.765 101.025) (width 0.4) (layer "F.Cu") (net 25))
 (segment (start 180.34 99.025) (end 181.645 100.33) (width 0.4) (layer "F.Cu") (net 23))
 (segment (start 178.435 99.025) (end 180.34 99.025) (width 0.4) (layer "F.Cu") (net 23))
 (segment (start 181.645 100.33) (end 183.515 100.33) (width 0.4) (layer "F.Cu") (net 23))
 (segment (start 178.435 97.025) (end 180.21 97.025) (width 0.4) (layer "F.Cu") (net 22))
 (segment (start 180.975 97.79) (end 183.515 97.79) (width 0.4) (layer "F.Cu") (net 22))
 (segment (start 180.21 97.025) (end 180.975 97.79) (width 0.4) (layer "F.Cu") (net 22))
 (segment (start 178.435 95.025) (end 183.29 95.025) (width 0.4) (layer "F.Cu") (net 21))
 (segment (start 183.29 95.025) (end 183.515 95.25) (width 0.4) (layer "F.Cu") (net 21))
 (segment (start 183.2 93.025) (end 183.515 92.71) (width 0.4) (layer "F.Cu") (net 20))
 (segment (start 178.435 93.025) (end 183.2 93.025) (width 0.4) (layer "F.Cu") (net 20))
 (segment (start 180.205 89.025) (end 181.6 87.63) (width 0.4) (layer "F.Cu") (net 17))
 (segment (start 178.435 89.025) (end 180.205 89.025) (width 0.4) (layer "F.Cu") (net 17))
 (segment (start 181.6 87.63) (end 183.515 87.63) (width 0.4) (layer "F.Cu") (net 17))
 (segment (start 178.435 87.025) (end 180.205 87.025) (width 0.4) (layer "F.Cu") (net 15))
 (segment (start 180.205 87.025) (end 182.14 85.09) (width 0.4) (layer "F.Cu") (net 15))
 (segment (start 182.14 85.09) (end 183.515 85.09) (width 0.4) (layer "F.Cu") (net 15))
 (segment (start 182.698334 82.55) (end 183.515 82.55) (width 0.4) (layer "F.Cu") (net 13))
 (segment (start 178.435 85.025) (end 180.223334 85.025) (width 0.4) (layer "F.Cu") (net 13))
 (segment (start 180.223334 85.025) (end 182.698334 82.55) (width 0.4) (layer "F.Cu") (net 13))
 (segment (start 178.435 83.025) (end 179.23 83.025) (width 0.4) (layer "F.Cu") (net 11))
 (segment (start 179.23 83.025) (end 182.245 80.01) (width 0.4) (layer "F.Cu") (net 11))
 (segment (start 182.245 80.01) (end 183.515 80.01) (width 0.4) (layer "F.Cu") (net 11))
 (segment (start 178.435 81.025) (end 179.143334 81.025) (width 0.4) (layer "F.Cu") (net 9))
 (segment (start 179.143334 81.025) (end 182.698334 77.47) (width 0.4) (layer "F.Cu") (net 9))
 (segment (start 182.698334 77.47) (end 183.515 77.47) (width 0.4) (layer "F.Cu") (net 9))
 (segment (start 180.975 76.653334) (end 182.698334 74.93) (width 0.4) (layer "F.Cu") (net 7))
 (segment (start 180.205 79.025) (end 180.975 78.255) (width 0.4) (layer "F.Cu") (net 7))
 (segment (start 182.698334 74.93) (end 183.515 74.93) (width 0.4) (layer "F.Cu") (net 7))
 (segment (start 180.975 78.255) (end 180.975 76.653334) (width 0.4) (layer "F.Cu") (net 7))
 (segment (start 178.435 79.025) (end 180.205 79.025) (width 0.4) (layer "F.Cu") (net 7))
 (segment (start 182.480001 72.39) (end 183.515 72.39) (width 0.4) (layer "F.Cu") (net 5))
 (segment (start 180.975 73.895001) (end 182.480001 72.39) (width 0.4) (layer "F.Cu") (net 5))
 (segment (start 179.515 77.025) (end 180.975 75.565) (width 0.4) (layer "F.Cu") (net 5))
 (segment (start 178.435 77.025) (end 179.515 77.025) (width 0.4) (layer "F.Cu") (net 5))
 (segment (start 180.975 75.565) (end 180.975 73.895001) (width 0.4) (layer "F.Cu") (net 5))
 (segment (start 178.435 75.025) (end 180.34 75.024999) (width 0.4) (layer "F.Cu") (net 3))
 (segment (start 182.698334 69.85) (end 183.515 69.85) (width 0.4) (layer "F.Cu") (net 3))
 (segment (start 180.34 75.024999) (end 180.34 72.208334) (width 0.4) (layer "F.Cu") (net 3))
 (segment (start 180.34 72.208334) (end 182.698334 69.85) (width 0.4) (layer "F.Cu") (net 3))
 (segment (start 180.975 67.71) (end 181.375 67.31) (width 0.4) (layer "F.Cu") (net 1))
 (segment (start 181.375 67.31) (end 183.515 67.31) (width 0.4) (layer "F.Cu") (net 1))
 (segment (start 180.975 70.485) (end 180.975 67.71) (width 0.4) (layer "F.Cu") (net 1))
 (segment (start 178.435 73.025) (end 180.975 70.485) (width 0.4) (layer "F.Cu") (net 1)))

